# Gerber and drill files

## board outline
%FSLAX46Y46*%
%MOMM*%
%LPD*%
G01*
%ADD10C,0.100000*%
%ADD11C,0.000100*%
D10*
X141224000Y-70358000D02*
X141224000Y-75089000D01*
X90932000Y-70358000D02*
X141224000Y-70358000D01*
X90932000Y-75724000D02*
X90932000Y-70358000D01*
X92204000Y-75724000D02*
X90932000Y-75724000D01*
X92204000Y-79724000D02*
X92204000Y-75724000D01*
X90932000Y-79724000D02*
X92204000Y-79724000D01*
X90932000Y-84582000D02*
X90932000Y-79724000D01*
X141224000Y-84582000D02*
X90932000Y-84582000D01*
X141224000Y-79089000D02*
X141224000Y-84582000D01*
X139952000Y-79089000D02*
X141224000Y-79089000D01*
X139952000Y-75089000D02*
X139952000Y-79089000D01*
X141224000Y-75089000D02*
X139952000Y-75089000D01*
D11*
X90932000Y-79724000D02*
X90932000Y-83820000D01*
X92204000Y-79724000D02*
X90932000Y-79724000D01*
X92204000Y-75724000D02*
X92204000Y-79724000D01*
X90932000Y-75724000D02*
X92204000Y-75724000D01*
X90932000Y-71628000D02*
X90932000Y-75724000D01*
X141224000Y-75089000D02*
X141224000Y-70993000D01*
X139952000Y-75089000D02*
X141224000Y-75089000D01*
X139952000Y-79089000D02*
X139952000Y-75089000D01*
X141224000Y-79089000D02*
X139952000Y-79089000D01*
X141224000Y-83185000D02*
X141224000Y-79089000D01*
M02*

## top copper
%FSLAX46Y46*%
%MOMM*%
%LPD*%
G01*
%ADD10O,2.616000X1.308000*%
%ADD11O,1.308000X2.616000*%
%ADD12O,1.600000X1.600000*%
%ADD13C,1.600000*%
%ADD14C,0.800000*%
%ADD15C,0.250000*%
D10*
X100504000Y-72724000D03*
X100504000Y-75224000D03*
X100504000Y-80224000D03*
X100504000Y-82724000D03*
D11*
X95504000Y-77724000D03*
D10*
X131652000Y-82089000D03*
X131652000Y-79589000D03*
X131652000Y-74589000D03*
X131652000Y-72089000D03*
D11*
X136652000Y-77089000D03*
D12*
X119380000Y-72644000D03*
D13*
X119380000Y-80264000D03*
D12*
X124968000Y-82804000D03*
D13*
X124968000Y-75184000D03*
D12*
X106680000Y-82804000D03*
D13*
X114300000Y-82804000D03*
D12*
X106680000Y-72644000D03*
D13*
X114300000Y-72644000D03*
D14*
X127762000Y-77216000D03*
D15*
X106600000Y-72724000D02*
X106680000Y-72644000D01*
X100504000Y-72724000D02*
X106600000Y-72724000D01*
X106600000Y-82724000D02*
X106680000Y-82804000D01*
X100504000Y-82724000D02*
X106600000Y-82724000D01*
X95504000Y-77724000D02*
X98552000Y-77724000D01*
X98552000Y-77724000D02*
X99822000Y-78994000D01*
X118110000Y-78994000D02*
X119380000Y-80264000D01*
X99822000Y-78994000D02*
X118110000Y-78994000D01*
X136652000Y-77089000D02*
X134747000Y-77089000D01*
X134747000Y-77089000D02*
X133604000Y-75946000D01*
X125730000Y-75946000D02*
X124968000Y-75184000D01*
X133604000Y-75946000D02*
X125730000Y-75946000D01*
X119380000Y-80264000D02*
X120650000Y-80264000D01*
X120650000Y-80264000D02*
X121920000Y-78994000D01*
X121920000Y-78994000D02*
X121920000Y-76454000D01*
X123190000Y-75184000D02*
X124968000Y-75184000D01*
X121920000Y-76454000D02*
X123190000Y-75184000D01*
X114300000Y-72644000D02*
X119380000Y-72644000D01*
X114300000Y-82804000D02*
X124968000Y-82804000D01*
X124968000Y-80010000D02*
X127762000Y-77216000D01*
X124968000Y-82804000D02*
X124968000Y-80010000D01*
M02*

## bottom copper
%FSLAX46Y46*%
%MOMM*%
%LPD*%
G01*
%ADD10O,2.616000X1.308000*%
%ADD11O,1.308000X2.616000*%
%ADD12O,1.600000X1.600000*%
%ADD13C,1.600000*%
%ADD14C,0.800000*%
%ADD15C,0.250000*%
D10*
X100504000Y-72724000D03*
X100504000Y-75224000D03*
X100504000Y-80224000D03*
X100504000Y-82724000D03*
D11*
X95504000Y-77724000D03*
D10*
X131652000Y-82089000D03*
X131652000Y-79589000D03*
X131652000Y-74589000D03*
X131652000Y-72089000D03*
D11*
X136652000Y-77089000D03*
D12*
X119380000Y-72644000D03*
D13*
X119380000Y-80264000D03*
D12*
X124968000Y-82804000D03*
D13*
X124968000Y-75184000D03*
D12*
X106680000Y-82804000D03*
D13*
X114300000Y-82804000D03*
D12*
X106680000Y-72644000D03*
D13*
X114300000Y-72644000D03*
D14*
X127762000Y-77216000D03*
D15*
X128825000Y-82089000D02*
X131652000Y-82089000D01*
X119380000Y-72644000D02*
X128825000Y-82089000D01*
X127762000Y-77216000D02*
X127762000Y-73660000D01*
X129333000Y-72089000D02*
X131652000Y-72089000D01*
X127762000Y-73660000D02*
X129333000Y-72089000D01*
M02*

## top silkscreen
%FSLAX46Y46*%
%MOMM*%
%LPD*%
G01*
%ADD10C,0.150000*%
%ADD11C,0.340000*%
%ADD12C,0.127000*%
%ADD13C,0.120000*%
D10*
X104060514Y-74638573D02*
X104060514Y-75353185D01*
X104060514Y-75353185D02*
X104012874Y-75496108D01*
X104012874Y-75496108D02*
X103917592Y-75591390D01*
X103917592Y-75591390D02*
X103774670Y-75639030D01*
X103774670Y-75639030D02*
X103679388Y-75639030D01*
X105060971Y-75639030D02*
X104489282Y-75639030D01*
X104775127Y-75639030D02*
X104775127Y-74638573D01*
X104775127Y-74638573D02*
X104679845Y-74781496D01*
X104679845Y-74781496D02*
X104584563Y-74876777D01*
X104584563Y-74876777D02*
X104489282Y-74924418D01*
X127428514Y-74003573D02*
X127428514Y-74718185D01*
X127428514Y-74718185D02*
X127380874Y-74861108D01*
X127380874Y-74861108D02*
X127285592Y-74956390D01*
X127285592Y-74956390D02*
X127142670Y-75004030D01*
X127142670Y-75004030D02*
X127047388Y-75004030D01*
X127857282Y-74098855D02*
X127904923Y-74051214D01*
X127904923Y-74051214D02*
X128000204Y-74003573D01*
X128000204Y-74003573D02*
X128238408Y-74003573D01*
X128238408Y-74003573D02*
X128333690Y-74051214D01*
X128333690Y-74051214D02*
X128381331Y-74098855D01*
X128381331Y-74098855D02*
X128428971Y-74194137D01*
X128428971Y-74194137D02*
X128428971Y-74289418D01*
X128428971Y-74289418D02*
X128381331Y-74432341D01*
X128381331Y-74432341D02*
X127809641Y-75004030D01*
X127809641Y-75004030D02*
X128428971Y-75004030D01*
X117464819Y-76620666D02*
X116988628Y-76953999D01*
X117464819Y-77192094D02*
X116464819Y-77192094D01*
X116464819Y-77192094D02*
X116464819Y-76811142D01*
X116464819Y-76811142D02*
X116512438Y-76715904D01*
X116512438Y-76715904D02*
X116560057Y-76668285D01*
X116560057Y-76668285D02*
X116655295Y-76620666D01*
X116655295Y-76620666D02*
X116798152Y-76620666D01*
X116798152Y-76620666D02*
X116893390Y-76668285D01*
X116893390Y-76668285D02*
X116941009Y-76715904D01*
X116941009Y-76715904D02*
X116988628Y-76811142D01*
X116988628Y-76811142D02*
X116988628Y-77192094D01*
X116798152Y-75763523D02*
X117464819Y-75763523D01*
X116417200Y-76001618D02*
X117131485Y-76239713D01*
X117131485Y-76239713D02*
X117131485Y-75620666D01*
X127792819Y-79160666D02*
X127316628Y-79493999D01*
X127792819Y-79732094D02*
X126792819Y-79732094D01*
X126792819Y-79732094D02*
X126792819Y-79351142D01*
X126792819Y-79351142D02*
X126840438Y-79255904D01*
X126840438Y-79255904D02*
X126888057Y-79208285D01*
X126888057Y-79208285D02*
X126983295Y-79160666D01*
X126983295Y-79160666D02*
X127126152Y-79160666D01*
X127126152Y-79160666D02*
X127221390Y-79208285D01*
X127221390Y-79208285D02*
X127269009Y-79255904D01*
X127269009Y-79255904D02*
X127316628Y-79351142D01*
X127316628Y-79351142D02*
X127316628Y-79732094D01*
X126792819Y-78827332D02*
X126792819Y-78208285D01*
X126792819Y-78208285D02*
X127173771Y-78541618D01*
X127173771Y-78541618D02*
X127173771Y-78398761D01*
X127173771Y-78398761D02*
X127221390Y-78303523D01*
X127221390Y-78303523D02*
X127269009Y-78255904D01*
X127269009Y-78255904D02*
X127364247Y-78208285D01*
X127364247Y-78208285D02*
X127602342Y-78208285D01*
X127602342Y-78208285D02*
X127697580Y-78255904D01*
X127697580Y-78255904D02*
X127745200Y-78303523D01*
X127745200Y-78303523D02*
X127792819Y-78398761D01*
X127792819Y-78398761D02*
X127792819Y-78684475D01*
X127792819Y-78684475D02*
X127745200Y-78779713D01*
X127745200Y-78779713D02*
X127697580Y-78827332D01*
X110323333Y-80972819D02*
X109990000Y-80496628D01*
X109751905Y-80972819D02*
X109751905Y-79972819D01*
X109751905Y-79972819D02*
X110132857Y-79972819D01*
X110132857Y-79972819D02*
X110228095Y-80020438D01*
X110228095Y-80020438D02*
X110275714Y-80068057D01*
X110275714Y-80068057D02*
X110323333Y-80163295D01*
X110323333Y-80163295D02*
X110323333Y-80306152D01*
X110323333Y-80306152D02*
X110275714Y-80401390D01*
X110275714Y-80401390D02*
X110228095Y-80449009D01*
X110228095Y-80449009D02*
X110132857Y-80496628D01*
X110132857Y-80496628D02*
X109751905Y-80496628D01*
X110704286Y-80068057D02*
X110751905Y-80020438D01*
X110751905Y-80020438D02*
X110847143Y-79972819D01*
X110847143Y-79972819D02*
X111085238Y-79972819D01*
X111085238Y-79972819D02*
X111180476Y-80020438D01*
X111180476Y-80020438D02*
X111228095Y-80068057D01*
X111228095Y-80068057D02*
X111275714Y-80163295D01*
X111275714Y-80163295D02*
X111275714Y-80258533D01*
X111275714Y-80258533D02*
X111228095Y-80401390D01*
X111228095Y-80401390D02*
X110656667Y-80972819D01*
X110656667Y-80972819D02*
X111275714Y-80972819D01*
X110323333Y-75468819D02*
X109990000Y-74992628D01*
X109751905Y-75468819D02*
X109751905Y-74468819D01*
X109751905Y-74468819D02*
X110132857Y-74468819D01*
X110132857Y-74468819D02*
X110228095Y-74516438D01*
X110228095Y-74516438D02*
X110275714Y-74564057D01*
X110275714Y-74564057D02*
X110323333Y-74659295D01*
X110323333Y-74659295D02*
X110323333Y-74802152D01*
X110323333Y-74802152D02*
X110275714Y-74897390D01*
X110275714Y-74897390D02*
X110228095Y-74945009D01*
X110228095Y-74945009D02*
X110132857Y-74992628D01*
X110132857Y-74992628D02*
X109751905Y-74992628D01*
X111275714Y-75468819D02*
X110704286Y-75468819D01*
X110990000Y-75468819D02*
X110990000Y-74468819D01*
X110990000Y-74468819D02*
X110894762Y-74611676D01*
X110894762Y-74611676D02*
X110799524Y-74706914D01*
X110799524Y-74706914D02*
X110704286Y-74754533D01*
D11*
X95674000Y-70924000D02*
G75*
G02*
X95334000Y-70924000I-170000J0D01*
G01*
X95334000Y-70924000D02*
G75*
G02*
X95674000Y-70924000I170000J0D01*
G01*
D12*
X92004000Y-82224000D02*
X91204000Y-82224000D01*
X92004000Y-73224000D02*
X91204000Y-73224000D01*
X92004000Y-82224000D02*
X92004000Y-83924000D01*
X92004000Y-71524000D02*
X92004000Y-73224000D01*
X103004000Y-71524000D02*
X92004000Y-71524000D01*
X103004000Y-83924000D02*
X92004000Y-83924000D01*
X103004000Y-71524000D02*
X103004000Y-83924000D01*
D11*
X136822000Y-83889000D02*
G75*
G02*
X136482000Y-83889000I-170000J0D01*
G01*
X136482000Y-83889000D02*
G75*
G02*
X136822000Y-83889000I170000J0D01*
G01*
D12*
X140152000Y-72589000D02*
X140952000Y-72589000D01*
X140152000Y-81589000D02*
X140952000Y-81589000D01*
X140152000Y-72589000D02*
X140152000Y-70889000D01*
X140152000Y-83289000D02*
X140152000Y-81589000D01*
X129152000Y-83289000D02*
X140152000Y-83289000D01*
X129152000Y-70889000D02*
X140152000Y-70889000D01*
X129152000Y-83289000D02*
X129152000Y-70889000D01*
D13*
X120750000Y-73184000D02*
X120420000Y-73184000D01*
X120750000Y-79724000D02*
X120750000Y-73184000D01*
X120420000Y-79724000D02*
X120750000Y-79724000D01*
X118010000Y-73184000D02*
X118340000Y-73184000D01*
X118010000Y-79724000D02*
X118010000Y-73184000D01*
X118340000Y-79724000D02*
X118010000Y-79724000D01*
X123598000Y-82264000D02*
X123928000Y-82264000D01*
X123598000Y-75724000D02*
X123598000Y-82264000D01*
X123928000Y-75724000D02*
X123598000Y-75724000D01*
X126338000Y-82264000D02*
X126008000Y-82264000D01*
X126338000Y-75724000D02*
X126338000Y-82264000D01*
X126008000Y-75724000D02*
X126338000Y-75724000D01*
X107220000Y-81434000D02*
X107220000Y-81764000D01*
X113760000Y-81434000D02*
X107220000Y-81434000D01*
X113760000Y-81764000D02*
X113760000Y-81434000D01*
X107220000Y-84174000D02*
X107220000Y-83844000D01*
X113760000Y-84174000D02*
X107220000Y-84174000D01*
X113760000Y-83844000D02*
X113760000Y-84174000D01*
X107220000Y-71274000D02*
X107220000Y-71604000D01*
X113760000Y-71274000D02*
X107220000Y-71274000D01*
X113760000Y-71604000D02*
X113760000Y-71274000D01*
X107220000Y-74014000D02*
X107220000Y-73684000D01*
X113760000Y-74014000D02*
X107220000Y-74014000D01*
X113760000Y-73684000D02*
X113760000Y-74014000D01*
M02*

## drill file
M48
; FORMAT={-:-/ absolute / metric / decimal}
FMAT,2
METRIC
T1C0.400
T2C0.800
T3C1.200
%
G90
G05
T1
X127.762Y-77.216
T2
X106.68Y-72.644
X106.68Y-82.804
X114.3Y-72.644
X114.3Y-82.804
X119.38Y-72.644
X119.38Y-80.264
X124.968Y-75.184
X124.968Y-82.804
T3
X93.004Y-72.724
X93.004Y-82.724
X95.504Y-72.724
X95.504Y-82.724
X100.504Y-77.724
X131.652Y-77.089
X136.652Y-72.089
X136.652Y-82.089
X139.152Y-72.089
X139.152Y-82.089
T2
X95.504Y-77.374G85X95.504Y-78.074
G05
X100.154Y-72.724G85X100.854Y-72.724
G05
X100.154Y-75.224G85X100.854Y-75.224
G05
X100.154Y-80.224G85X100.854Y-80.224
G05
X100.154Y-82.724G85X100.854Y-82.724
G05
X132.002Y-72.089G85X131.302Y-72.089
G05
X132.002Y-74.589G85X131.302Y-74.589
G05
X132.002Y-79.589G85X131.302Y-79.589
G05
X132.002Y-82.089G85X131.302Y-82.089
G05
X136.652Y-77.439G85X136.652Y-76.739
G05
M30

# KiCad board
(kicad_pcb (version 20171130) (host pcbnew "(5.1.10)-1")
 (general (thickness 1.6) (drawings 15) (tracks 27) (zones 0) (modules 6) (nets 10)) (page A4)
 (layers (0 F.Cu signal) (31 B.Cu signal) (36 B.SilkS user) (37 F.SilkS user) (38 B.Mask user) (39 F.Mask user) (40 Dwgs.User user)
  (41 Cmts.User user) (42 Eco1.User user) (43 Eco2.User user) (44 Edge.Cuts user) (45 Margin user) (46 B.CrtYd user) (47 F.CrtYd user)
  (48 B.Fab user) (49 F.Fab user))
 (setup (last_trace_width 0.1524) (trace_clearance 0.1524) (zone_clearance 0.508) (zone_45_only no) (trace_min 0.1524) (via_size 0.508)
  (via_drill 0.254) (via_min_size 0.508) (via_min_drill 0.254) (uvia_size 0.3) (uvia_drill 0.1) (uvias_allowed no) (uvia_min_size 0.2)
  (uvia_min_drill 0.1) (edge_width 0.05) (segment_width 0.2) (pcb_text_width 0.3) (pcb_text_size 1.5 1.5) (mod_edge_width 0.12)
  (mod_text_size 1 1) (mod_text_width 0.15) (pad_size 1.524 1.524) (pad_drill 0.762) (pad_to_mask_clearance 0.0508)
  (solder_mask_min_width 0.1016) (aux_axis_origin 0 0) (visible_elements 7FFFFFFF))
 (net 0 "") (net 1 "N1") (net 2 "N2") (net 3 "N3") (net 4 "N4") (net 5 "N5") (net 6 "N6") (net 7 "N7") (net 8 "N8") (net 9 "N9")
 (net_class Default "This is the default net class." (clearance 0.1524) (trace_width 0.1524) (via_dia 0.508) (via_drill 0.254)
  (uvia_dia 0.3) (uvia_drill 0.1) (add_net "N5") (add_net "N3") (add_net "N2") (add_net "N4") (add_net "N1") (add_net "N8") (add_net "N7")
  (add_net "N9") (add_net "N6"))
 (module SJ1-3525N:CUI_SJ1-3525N (layer F.Cu) (at 95.504 77.724)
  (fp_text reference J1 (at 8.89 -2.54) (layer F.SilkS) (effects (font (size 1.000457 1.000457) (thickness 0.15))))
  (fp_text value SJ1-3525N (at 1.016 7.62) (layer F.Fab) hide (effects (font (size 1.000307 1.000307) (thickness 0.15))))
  (fp_circle (center 0 -6.8) (end 0.17 -6.8) (layer F.SilkS) (width 0.34))
  (fp_line (start -3.5 4.5) (end -4.3 4.5) (layer F.SilkS) (width 0.127))
  (fp_line (start -3.5 -4.5) (end -4.3 -4.5) (layer F.SilkS) (width 0.127))
  (fp_line (start -3.5 4.5) (end -3.5 6.2) (layer F.SilkS) (width 0.127))
  (fp_line (start -3.5 -6.2) (end -3.5 -4.5) (layer F.SilkS) (width 0.127))
  (fp_line (start 7.5 -6.2) (end -3.5 -6.2) (layer F.SilkS) (width 0.127))
  (fp_line (start 7.5 6.2) (end -3.5 6.2) (layer F.SilkS) (width 0.127))
  (fp_line (start 7.5 -6.2) (end 7.5 6.2) (layer F.SilkS) (width 0.127))
  (fp_line (start -4.572 2) (end -4.572 6.096) (layer Edge.Cuts) (width 0.0001))
  (fp_line (start -3.3 2) (end -4.572 2) (layer Edge.Cuts) (width 0.0001))
  (fp_line (start -3.3 -2) (end -3.3 2) (layer Edge.Cuts) (width 0.0001))
  (fp_line (start -4.572 -2) (end -3.3 -2) (layer Edge.Cuts) (width 0.0001))
  (fp_line (start -4.572 -6.096) (end -4.572 -2) (layer Edge.Cuts) (width 0.0001))
  (pad None np_thru_hole circle (at 0 5) (size 1.2 1.2) (drill 1.2) (layers *.Cu *.Mask))
  (pad None np_thru_hole circle (at -2.5 5) (size 1.2 1.2) (drill 1.2) (layers *.Cu *.Mask))
  (pad None np_thru_hole circle (at 5 0) (size 1.2 1.2) (drill 1.2) (layers *.Cu *.Mask))
  (pad None np_thru_hole circle (at 0 -5) (size 1.2 1.2) (drill 1.2) (layers *.Cu *.Mask))
  (pad None np_thru_hole circle (at -2.5 -5) (size 1.2 1.2) (drill 1.2) (layers *.Cu *.Mask))
  (pad 3 thru_hole oval (at 5 -5) (size 2.616 1.308) (drill oval 1.5 0.8) (layers *.Cu *.Mask) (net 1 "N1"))
  (pad 11 thru_hole oval (at 5 -2.5) (size 2.616 1.308) (drill oval 1.5 0.8) (layers *.Cu *.Mask) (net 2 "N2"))
  (pad 10 thru_hole oval (at 5 2.5) (size 2.616 1.308) (drill oval 1.5 0.8) (layers *.Cu *.Mask) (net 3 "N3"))
  (pad 2 thru_hole oval (at 5 5) (size 2.616 1.308) (drill oval 1.5 0.8) (layers *.Cu *.Mask) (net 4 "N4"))
  (pad 1 thru_hole oval (at 0 0) (size 1.308 2.616) (drill oval 0.8 1.5) (layers *.Cu *.Mask) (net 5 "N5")))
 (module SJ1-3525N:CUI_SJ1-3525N (layer F.Cu) (at 136.652 77.089 180)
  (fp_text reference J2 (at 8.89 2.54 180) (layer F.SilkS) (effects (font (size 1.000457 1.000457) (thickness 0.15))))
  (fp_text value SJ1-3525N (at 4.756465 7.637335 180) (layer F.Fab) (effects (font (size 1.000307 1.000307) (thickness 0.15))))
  (fp_circle (center 0 -6.8) (end 0.17 -6.8) (layer F.SilkS) (width 0.34))
  (fp_line (start -3.5 4.5) (end -4.3 4.5) (layer F.SilkS) (width 0.127))
  (fp_line (start -3.5 -4.5) (end -4.3 -4.5) (layer F.SilkS) (width 0.127))
  (fp_line (start -3.5 4.5) (end -3.5 6.2) (layer F.SilkS) (width 0.127))
  (fp_line (start -3.5 -6.2) (end -3.5 -4.5) (layer F.SilkS) (width 0.127))
  (fp_line (start 7.5 -6.2) (end -3.5 -6.2) (layer F.SilkS) (width 0.127))
  (fp_line (start 7.5 6.2) (end -3.5 6.2) (layer F.SilkS) (width 0.127))
  (fp_line (start 7.5 -6.2) (end 7.5 6.2) (layer F.SilkS) (width 0.127))
  (fp_line (start -4.572 2) (end -4.572 6.096) (layer Edge.Cuts) (width 0.0001))
  (fp_line (start -3.3 2) (end -4.572 2) (layer Edge.Cuts) (width 0.0001))
  (fp_line (start -3.3 -2) (end -3.3 2) (layer Edge.Cuts) (width 0.0001))
  (fp_line (start -4.572 -2) (end -3.3 -2) (layer Edge.Cuts) (width 0.0001))
  (fp_line (start -4.572 -6.096) (end -4.572 -2) (layer Edge.Cuts) (width 0.0001))
  (pad None np_thru_hole circle (at 0 5 180) (size 1.2 1.2) (drill 1.2) (layers *.Cu *.Mask))
  (pad None np_thru_hole circle (at -2.5 5 180) (size 1.2 1.2) (drill 1.2) (layers *.Cu *.Mask))
  (pad None np_thru_hole circle (at 5 0 180) (size 1.2 1.2) (drill 1.2) (layers *.Cu *.Mask))
  (pad None np_thru_hole circle (at 0 -5 180) (size 1.2 1.2) (drill 1.2) (layers *.Cu *.Mask))
  (pad None np_thru_hole circle (at -2.5 -5 180) (size 1.2 1.2) (drill 1.2) (layers *.Cu *.Mask))
  (pad 3 thru_hole oval (at 5 -5 180) (size 2.616 1.308) (drill oval 1.5 0.8) (layers *.Cu *.Mask) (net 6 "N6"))
  (pad 11 thru_hole oval (at 5 -2.5 180) (size 2.616 1.308) (drill oval 1.5 0.8) (layers *.Cu *.Mask) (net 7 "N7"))
  (pad 10 thru_hole oval (at 5 2.5 180) (size 2.616 1.308) (drill oval 1.5 0.8) (layers *.Cu *.Mask) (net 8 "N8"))
  (pad 2 thru_hole oval (at 5 5 180) (size 2.616 1.308) (drill oval 1.5 0.8) (layers *.Cu *.Mask) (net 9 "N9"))
  (pad 1 thru_hole oval (at 0 0 180) (size 1.308 2.616) (drill oval 0.8 1.5) (layers *.Cu *.Mask) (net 5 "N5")))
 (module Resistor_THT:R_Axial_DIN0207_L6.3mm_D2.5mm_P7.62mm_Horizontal (layer F.Cu) (at 119.38 80.264 90)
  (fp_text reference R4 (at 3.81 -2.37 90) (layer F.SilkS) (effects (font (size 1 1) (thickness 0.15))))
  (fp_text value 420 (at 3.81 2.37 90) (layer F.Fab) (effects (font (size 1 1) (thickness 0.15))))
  (fp_line (start 7.08 1.37) (end 7.08 1.04) (layer F.SilkS) (width 0.12))
  (fp_line (start 0.54 1.37) (end 7.08 1.37) (layer F.SilkS) (width 0.12))
  (fp_line (start 0.54 1.04) (end 0.54 1.37) (layer F.SilkS) (width 0.12))
  (fp_line (start 7.08 -1.37) (end 7.08 -1.04) (layer F.SilkS) (width 0.12))
  (fp_line (start 0.54 -1.37) (end 7.08 -1.37) (layer F.SilkS) (width 0.12))
  (fp_line (start 0.54 -1.04) (end 0.54 -1.37) (layer F.SilkS) (width 0.12))
  (pad 2 thru_hole oval (at 7.62 0 90) (size 1.6 1.6) (drill 0.8) (layers *.Cu *.Mask) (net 6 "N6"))
  (pad 1 thru_hole circle (at 0 0 90) (size 1.6 1.6) (drill 0.8) (layers *.Cu *.Mask) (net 5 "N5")))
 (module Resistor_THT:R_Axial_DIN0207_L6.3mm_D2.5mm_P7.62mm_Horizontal (layer F.Cu) (at 124.968 75.184 270)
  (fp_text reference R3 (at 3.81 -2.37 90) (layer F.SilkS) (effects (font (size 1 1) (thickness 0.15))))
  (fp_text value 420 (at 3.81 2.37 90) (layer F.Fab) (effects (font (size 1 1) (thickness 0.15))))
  (fp_line (start 7.08 1.37) (end 7.08 1.04) (layer F.SilkS) (width 0.12))
  (fp_line (start 0.54 1.37) (end 7.08 1.37) (layer F.SilkS) (width 0.12))
  (fp_line (start 0.54 1.04) (end 0.54 1.37) (layer F.SilkS) (width 0.12))
  (fp_line (start 7.08 -1.37) (end 7.08 -1.04) (layer F.SilkS) (width 0.12))
  (fp_line (start 0.54 -1.37) (end 7.08 -1.37) (layer F.SilkS) (width 0.12))
  (fp_line (start 0.54 -1.04) (end 0.54 -1.37) (layer F.SilkS) (width 0.12))
  (pad 2 thru_hole oval (at 7.62 0 270) (size 1.6 1.6) (drill 0.8) (layers *.Cu *.Mask) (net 9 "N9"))
  (pad 1 thru_hole circle (at 0 0 270) (size 1.6 1.6) (drill 0.8) (layers *.Cu *.Mask) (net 5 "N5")))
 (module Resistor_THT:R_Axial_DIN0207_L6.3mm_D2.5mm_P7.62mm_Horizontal (layer F.Cu) (at 114.3 82.804 180)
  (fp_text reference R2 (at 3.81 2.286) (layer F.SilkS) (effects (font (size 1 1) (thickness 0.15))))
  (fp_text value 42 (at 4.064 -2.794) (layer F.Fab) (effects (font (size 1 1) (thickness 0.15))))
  (fp_line (start 7.08 1.37) (end 7.08 1.04) (layer F.SilkS) (width 0.12))
  (fp_line (start 0.54 1.37) (end 7.08 1.37) (layer F.SilkS) (width 0.12))
  (fp_line (start 0.54 1.04) (end 0.54 1.37) (layer F.SilkS) (width 0.12))
  (fp_line (start 7.08 -1.37) (end 7.08 -1.04) (layer F.SilkS) (width 0.12))
  (fp_line (start 0.54 -1.37) (end 7.08 -1.37) (layer F.SilkS) (width 0.12))
  (fp_line (start 0.54 -1.04) (end 0.54 -1.37) (layer F.SilkS) (width 0.12))
  (pad 2 thru_hole oval (at 7.62 0 180) (size 1.6 1.6) (drill 0.8) (layers *.Cu *.Mask) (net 4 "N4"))
  (pad 1 thru_hole circle (at 0 0 180) (size 1.6 1.6) (drill 0.8) (layers *.Cu *.Mask) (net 9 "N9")))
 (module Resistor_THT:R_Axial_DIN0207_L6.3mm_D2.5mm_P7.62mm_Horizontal (layer F.Cu) (at 114.3 72.644 180)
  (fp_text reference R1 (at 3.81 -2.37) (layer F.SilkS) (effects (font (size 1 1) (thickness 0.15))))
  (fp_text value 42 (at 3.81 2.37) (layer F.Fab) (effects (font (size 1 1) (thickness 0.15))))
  (fp_line (start 7.08 1.37) (end 7.08 1.04) (layer F.SilkS) (width 0.12))
  (fp_line (start 0.54 1.37) (end 7.08 1.37) (layer F.SilkS) (width 0.12))
  (fp_line (start 0.54 1.04) (end 0.54 1.37) (layer F.SilkS) (width 0.12))
  (fp_line (start 7.08 -1.37) (end 7.08 -1.04) (layer F.SilkS) (width 0.12))
  (fp_line (start 0.54 -1.37) (end 7.08 -1.37) (layer F.SilkS) (width 0.12))
  (fp_line (start 0.54 -1.04) (end 0.54 -1.37) (layer F.SilkS) (width 0.12))
  (pad 2 thru_hole oval (at 7.62 0 180) (size 1.6 1.6) (drill 0.8) (layers *.Cu *.Mask) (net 1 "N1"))
  (pad 1 thru_hole circle (at 0 0 180) (size 1.6 1.6) (drill 0.8) (layers *.Cu *.Mask) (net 6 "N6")))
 (gr_line (start 141.224 70.358) (end 141.224 75.089) (layer Edge.Cuts) (width 0.1))
 (gr_line (start 90.932 70.358) (end 141.224 70.358) (layer Edge.Cuts) (width 0.1))
 (gr_line (start 90.932 75.724) (end 90.932 70.358) (layer Edge.Cuts) (width 0.1))
 (gr_line (start 92.204 75.724) (end 90.932 75.724) (layer Edge.Cuts) (width 0.1))
 (gr_line (start 92.204 79.724) (end 92.204 75.724) (layer Edge.Cuts) (width 0.1))
 (gr_line (start 90.932 79.724) (end 92.204 79.724) (layer Edge.Cuts) (width 0.1))
 (gr_line (start 90.932 84.582) (end 90.932 79.724) (layer Edge.Cuts) (width 0.1))
 (gr_line (start 141.224 84.582) (end 90.932 84.582) (layer Edge.Cuts) (width 0.1))
 (gr_line (start 141.224 79.089) (end 141.224 84.582) (layer Edge.Cuts) (width 0.1))
 (gr_line (start 139.952 79.089) (end 141.224 79.089) (layer Edge.Cuts) (width 0.1))
 (gr_line (start 139.952 75.089) (end 139.952 79.089) (layer Edge.Cuts) (width 0.1))
 (gr_line (start 141.224 75.089) (end 139.952 75.089) (layer Edge.Cuts) (width 0.1))
 (segment (start 106.6 72.724) (end 106.68 72.644) (width 0.25) (layer F.Cu) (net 1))
 (segment (start 100.504 72.724) (end 106.6 72.724) (width 0.25) (layer F.Cu) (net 1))
 (segment (start 106.6 82.724) (end 106.68 82.804) (width 0.25) (layer F.Cu) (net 4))
 (segment (start 100.504 82.724) (end 106.6 82.724) (width 0.25) (layer F.Cu) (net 4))
 (segment (start 95.504 77.724) (end 98.552 77.724) (width 0.25) (layer F.Cu) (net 5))
 (segment (start 98.552 77.724) (end 99.822 78.994) (width 0.25) (layer F.Cu) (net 5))
 (segment (start 118.11 78.994) (end 119.38 80.264) (width 0.25) (layer F.Cu) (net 5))
 (segment (start 99.822 78.994) (end 118.11 78.994) (width 0.25) (layer F.Cu) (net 5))
 (segment (start 136.652 77.089) (end 134.747 77.089) (width 0.25) (layer F.Cu) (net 5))
 (segment (start 134.747 77.089) (end 133.604 75.946) (width 0.25) (layer F.Cu) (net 5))
 (segment (start 125.73 75.946) (end 124.968 75.184) (width 0.25) (layer F.Cu) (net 5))
 (segment (start 133.604 75.946) (end 125.73 75.946) (width 0.25) (layer F.Cu) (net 5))
 (segment (start 119.38 80.264) (end 120.65 80.264) (width 0.25) (layer F.Cu) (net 5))
 (segment (start 120.65 80.264) (end 121.92 78.994) (width 0.25) (layer F.Cu) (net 5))
 (segment (start 121.92 78.994) (end 121.92 76.454) (width 0.25) (layer F.Cu) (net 5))
 (segment (start 123.19 75.184) (end 124.968 75.184) (width 0.25) (layer F.Cu) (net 5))
 (segment (start 121.92 76.454) (end 123.19 75.184) (width 0.25) (layer F.Cu) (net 5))
 (segment (start 114.3 72.644) (end 119.38 72.644) (width 0.25) (layer F.Cu) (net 6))
 (segment (start 128.825 82.089) (end 131.652 82.089) (width 0.25) (layer B.Cu) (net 6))
 (segment (start 119.38 72.644) (end 128.825 82.089) (width 0.25) (layer B.Cu) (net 6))
 (segment (start 114.3 82.804) (end 124.968 82.804) (width 0.25) (layer F.Cu) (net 9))
 (via (at 127.762 77.216) (size 0.8) (drill 0.4) (layers F.Cu B.Cu) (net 9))
 (segment (start 124.968 80.01) (end 127.762 77.216) (width 0.25) (layer F.Cu) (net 9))
 (segment (start 124.968 82.804) (end 124.968 80.01) (width 0.25) (layer F.Cu) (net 9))
 (segment (start 127.762 77.216) (end 127.762 73.66) (width 0.25) (layer B.Cu) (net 9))
 (segment (start 129.333 72.089) (end 131.652 72.089) (width 0.25) (layer B.Cu) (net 9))
 (segment (start 127.762 73.66) (end 129.333 72.089) (width 0.25) (layer B.Cu) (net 9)))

